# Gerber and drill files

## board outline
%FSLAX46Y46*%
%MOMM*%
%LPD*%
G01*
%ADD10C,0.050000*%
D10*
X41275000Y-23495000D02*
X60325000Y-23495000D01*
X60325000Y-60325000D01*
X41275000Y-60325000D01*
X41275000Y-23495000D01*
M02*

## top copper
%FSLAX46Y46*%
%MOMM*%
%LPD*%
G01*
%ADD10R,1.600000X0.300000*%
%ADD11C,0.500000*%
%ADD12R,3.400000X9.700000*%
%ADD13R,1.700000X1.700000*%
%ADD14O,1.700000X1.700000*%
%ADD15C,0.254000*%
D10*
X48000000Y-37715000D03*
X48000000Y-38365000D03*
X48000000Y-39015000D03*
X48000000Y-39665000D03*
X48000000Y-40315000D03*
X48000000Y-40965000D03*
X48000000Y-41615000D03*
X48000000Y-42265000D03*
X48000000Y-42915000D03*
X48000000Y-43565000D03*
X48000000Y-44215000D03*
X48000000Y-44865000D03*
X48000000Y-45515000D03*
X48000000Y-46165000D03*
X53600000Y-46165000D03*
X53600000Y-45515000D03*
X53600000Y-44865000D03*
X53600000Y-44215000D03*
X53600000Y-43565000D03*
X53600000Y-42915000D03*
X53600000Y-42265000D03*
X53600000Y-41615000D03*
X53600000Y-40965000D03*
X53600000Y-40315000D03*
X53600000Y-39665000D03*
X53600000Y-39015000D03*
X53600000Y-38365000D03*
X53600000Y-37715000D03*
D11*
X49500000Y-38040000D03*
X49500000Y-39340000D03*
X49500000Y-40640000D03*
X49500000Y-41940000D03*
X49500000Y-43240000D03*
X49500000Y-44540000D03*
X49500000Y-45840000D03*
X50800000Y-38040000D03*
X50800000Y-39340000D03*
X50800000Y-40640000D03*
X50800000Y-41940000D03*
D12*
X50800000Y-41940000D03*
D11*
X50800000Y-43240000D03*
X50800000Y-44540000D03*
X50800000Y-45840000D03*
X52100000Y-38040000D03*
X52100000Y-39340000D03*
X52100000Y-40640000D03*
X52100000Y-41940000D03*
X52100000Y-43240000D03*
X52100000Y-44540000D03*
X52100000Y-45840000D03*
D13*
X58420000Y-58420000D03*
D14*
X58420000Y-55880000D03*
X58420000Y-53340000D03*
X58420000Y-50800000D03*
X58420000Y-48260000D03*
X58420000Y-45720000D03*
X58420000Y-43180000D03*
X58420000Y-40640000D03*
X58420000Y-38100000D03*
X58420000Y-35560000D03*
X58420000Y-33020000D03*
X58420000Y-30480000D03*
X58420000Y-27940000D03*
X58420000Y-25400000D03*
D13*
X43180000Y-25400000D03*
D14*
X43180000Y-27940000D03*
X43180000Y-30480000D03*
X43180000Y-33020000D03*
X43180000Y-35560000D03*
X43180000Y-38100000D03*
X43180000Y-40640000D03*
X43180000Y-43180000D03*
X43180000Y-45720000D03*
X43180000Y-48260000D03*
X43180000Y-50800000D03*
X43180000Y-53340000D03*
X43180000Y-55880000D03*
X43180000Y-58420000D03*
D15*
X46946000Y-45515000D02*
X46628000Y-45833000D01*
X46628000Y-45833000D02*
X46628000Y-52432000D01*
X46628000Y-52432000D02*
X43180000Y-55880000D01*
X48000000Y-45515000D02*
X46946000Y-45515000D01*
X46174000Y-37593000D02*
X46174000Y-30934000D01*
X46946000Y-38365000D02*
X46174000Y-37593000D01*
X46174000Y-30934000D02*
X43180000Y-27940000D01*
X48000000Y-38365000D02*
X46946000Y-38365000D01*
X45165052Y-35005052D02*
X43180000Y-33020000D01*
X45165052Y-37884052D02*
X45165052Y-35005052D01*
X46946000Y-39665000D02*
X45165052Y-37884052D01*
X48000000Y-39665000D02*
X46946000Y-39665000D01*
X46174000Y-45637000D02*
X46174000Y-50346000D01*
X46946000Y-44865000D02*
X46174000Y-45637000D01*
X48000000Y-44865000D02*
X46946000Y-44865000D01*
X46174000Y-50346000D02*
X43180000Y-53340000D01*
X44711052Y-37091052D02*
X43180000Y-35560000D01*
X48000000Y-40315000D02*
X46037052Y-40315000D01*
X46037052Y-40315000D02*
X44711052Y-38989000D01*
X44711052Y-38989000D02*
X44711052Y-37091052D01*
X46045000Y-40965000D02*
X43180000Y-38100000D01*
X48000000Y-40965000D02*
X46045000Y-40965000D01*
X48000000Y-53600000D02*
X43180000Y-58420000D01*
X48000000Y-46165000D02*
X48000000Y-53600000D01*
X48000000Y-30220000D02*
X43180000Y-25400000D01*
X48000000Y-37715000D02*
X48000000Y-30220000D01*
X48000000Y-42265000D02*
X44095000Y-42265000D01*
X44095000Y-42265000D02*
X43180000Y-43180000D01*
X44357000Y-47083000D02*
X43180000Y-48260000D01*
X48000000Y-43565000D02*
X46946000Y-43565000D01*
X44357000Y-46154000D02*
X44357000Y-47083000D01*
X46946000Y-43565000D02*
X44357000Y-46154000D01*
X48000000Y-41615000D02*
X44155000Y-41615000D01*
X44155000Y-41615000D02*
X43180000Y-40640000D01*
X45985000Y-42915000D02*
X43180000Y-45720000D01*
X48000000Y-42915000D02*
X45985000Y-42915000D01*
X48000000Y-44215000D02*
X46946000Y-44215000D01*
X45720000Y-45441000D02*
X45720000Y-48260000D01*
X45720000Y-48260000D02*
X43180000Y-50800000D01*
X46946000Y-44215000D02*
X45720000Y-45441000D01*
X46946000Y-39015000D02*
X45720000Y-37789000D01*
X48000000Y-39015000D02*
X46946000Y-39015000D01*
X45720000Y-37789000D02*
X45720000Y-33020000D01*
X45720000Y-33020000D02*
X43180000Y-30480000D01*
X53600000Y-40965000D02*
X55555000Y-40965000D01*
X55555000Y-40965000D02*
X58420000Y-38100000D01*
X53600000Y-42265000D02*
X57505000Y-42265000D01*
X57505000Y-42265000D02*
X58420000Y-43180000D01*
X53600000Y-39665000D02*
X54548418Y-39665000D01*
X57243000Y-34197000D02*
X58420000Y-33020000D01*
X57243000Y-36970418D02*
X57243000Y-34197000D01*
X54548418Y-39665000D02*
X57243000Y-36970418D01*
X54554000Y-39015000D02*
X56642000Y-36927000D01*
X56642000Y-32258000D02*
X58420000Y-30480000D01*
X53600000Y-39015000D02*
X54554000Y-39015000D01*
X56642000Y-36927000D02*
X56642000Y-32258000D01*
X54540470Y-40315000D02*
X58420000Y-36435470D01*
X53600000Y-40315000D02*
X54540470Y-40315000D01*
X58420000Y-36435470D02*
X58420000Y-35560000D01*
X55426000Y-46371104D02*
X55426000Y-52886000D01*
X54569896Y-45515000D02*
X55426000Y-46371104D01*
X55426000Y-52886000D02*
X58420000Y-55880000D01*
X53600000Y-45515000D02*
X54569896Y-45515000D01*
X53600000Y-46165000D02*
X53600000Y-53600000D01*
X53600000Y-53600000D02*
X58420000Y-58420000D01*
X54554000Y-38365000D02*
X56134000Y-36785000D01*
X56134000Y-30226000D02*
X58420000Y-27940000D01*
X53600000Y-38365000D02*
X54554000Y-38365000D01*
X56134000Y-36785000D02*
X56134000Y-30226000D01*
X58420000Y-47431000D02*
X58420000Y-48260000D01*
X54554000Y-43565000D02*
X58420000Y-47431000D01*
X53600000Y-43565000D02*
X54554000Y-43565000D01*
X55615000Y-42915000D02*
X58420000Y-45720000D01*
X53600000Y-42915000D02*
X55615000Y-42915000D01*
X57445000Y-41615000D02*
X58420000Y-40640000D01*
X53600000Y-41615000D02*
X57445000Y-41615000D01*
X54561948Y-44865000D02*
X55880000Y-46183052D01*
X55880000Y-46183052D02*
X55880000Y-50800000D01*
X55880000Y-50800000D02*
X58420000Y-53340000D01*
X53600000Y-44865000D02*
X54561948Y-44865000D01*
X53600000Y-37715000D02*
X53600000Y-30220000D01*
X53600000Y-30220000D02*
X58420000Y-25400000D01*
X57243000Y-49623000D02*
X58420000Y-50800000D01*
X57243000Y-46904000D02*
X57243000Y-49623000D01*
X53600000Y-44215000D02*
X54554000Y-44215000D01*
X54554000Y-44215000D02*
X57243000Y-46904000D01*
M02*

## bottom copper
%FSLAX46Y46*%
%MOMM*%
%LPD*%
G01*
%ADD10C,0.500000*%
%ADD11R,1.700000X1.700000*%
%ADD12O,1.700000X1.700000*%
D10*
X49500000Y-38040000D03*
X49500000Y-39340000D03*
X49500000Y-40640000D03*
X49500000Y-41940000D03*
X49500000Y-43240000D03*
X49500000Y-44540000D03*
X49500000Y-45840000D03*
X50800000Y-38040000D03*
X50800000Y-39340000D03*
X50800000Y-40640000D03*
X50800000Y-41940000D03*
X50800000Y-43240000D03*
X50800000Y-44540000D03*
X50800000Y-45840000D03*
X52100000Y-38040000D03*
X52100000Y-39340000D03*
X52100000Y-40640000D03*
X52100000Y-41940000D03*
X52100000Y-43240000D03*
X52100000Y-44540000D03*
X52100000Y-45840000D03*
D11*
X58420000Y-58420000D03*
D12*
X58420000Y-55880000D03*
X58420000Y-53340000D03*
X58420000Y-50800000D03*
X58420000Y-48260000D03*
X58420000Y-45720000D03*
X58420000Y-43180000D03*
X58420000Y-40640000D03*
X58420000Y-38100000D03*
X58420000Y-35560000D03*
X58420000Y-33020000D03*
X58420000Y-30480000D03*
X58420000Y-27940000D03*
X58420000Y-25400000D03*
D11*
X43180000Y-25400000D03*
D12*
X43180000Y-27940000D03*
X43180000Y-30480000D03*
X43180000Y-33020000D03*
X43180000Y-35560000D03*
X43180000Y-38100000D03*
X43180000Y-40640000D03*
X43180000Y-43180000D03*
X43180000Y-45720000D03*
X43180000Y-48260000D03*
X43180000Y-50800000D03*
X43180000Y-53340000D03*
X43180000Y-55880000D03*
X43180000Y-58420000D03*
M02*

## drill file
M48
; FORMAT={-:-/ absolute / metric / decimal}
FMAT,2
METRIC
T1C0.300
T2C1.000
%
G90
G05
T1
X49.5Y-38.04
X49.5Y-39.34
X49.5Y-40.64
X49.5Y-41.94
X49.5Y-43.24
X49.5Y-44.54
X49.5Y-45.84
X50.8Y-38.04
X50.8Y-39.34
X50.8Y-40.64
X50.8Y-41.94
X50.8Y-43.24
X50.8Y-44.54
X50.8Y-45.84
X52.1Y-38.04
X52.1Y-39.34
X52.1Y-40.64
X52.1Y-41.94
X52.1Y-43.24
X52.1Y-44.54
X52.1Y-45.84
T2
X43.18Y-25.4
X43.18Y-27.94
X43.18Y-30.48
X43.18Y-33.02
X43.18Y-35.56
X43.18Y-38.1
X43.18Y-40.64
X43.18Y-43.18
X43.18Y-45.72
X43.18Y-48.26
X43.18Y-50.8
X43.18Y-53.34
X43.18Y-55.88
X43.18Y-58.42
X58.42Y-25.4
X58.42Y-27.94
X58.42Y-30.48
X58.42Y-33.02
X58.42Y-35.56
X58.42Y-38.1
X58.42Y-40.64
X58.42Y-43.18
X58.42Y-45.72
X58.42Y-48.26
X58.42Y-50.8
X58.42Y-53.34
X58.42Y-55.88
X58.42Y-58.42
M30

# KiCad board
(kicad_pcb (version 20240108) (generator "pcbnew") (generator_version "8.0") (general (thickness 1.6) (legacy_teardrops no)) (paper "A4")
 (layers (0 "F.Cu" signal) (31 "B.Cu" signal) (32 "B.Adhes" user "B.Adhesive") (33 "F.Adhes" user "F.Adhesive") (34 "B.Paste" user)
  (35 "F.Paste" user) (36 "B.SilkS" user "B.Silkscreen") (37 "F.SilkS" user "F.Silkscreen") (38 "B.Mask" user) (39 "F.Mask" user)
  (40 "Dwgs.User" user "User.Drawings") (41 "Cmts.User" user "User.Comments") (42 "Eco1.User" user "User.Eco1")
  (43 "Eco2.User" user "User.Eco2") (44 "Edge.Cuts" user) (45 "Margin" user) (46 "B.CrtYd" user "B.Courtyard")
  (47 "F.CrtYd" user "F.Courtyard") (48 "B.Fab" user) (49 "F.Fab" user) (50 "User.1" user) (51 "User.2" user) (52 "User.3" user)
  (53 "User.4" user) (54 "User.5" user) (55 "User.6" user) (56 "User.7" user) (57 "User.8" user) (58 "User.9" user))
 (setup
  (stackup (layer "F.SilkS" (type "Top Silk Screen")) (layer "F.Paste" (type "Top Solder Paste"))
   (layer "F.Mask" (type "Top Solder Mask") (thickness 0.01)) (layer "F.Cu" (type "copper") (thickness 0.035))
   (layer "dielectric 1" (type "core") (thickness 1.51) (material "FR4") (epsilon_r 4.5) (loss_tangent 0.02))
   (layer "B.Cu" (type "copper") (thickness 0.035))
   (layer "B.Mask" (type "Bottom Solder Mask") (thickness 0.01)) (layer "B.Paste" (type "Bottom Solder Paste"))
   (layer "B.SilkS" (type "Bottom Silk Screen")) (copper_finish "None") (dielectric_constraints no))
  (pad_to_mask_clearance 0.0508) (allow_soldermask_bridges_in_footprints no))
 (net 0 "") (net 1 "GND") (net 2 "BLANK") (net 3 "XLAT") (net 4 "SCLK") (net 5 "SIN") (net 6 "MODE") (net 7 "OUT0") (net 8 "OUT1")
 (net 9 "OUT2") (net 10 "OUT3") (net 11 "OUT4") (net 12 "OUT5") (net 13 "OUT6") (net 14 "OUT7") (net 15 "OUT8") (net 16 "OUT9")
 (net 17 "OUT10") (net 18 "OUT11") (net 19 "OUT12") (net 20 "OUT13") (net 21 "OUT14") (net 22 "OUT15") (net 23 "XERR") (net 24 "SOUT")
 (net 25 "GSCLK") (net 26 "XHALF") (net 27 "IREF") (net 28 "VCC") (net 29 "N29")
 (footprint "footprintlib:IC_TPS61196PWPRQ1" (layer "F.Cu") (at 50.8 41.94)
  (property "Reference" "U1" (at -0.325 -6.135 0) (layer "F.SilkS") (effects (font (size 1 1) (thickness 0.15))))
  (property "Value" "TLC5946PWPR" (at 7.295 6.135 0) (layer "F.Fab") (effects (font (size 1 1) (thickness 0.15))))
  (pad "1" smd rect (at -2.8 -4.225) (size 1.6 0.3) (layers "F.Cu") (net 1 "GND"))
  (pad "2" smd rect (at -2.8 -3.575) (size 1.6 0.3) (layers "F.Cu") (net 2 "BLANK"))
  (pad "3" smd rect (at -2.8 -2.925) (size 1.6 0.3) (layers "F.Cu") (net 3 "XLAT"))
  (pad "4" smd rect (at -2.8 -2.275) (size 1.6 0.3) (layers "F.Cu") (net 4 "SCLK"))
  (pad "5" smd rect (at -2.8 -1.625) (size 1.6 0.3) (layers "F.Cu") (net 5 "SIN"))
  (pad "6" smd rect (at -2.8 -0.975) (size 1.6 0.3) (layers "F.Cu") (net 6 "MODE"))
  (pad "7" smd rect (at -2.8 -0.325) (size 1.6 0.3) (layers "F.Cu") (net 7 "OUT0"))
  (pad "8" smd rect (at -2.8 0.325) (size 1.6 0.3) (layers "F.Cu") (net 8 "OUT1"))
  (pad "9" smd rect (at -2.8 0.975) (size 1.6 0.3) (layers "F.Cu") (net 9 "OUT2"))
  (pad "10" smd rect (at -2.8 1.625) (size 1.6 0.3) (layers "F.Cu") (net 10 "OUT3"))
  (pad "11" smd rect (at -2.8 2.275) (size 1.6 0.3) (layers "F.Cu") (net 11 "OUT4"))
  (pad "12" smd rect (at -2.8 2.925) (size 1.6 0.3) (layers "F.Cu") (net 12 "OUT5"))
  (pad "13" smd rect (at -2.8 3.575) (size 1.6 0.3) (layers "F.Cu") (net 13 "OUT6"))
  (pad "14" smd rect (at -2.8 4.225) (size 1.6 0.3) (layers "F.Cu") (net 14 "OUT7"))
  (pad "15" smd rect (at 2.8 4.225) (size 1.6 0.3) (layers "F.Cu") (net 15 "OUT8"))
  (pad "16" smd rect (at 2.8 3.575) (size 1.6 0.3) (layers "F.Cu") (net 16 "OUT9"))
  (pad "17" smd rect (at 2.8 2.925) (size 1.6 0.3) (layers "F.Cu") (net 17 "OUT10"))
  (pad "18" smd rect (at 2.8 2.275) (size 1.6 0.3) (layers "F.Cu") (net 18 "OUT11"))
  (pad "19" smd rect (at 2.8 1.625) (size 1.6 0.3) (layers "F.Cu") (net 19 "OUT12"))
  (pad "20" smd rect (at 2.8 0.975) (size 1.6 0.3) (layers "F.Cu") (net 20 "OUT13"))
  (pad "21" smd rect (at 2.8 0.325) (size 1.6 0.3) (layers "F.Cu") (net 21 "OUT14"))
  (pad "22" smd rect (at 2.8 -0.325) (size 1.6 0.3) (layers "F.Cu") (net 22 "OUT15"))
  (pad "23" smd rect (at 2.8 -0.975) (size 1.6 0.3) (layers "F.Cu") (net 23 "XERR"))
  (pad "24" smd rect (at 2.8 -1.625) (size 1.6 0.3) (layers "F.Cu") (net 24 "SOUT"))
  (pad "25" smd rect (at 2.8 -2.275) (size 1.6 0.3) (layers "F.Cu") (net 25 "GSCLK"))
  (pad "26" smd rect (at 2.8 -2.925) (size 1.6 0.3) (layers "F.Cu") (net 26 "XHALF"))
  (pad "27" smd rect (at 2.8 -3.575) (size 1.6 0.3) (layers "F.Cu") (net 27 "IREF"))
  (pad "28" smd rect (at 2.8 -4.225) (size 1.6 0.3) (layers "F.Cu") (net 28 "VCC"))
  (pad "29" thru_hole circle (at -1.3 -3.9) (size 0.5 0.5) (drill 0.3) (layers "*.Cu") (remove_unused_layers no) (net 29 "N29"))
  (pad "29" thru_hole circle (at -1.3 -2.6) (size 0.5 0.5) (drill 0.3) (layers "*.Cu") (remove_unused_layers no) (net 29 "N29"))
  (pad "29" thru_hole circle (at -1.3 -1.3) (size 0.5 0.5) (drill 0.3) (layers "*.Cu") (remove_unused_layers no) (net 29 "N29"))
  (pad "29" thru_hole circle (at -1.3 0) (size 0.5 0.5) (drill 0.3) (layers "*.Cu") (remove_unused_layers no) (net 29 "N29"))
  (pad "29" thru_hole circle (at -1.3 1.3) (size 0.5 0.5) (drill 0.3) (layers "*.Cu") (remove_unused_layers no) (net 29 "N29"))
  (pad "29" thru_hole circle (at -1.3 2.6) (size 0.5 0.5) (drill 0.3) (layers "*.Cu") (remove_unused_layers no) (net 29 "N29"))
  (pad "29" thru_hole circle (at -1.3 3.9) (size 0.5 0.5) (drill 0.3) (layers "*.Cu") (remove_unused_layers no) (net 29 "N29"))
  (pad "29" thru_hole circle (at 0 -3.9) (size 0.5 0.5) (drill 0.3) (layers "*.Cu") (remove_unused_layers no) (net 29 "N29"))
  (pad "29" thru_hole circle (at 0 -2.6) (size 0.5 0.5) (drill 0.3) (layers "*.Cu") (remove_unused_layers no) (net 29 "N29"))
  (pad "29" thru_hole circle (at 0 -1.3) (size 0.5 0.5) (drill 0.3) (layers "*.Cu") (remove_unused_layers no) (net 29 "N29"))
  (pad "29" thru_hole circle (at 0 0) (size 0.5 0.5) (drill 0.3) (layers "*.Cu") (remove_unused_layers no) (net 29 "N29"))
  (pad "29" smd rect (at 0 0) (size 3.4 9.7) (layers "F.Cu") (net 29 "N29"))
  (pad "29" thru_hole circle (at 0 1.3) (size 0.5 0.5) (drill 0.3) (layers "*.Cu") (remove_unused_layers no) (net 29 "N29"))
  (pad "29" thru_hole circle (at 0 2.6) (size 0.5 0.5) (drill 0.3) (layers "*.Cu") (remove_unused_layers no) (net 29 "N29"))
  (pad "29" thru_hole circle (at 0 3.9) (size 0.5 0.5) (drill 0.3) (layers "*.Cu") (remove_unused_layers no) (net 29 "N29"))
  (pad "29" thru_hole circle (at 1.3 -3.9) (size 0.5 0.5) (drill 0.3) (layers "*.Cu") (remove_unused_layers no) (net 29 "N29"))
  (pad "29" thru_hole circle (at 1.3 -2.6) (size 0.5 0.5) (drill 0.3) (layers "*.Cu") (remove_unused_layers no) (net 29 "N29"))
  (pad "29" thru_hole circle (at 1.3 -1.3) (size 0.5 0.5) (drill 0.3) (layers "*.Cu") (remove_unused_layers no) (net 29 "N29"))
  (pad "29" thru_hole circle (at 1.3 0) (size 0.5 0.5) (drill 0.3) (layers "*.Cu") (remove_unused_layers no) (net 29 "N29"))
  (pad "29" thru_hole circle (at 1.3 1.3) (size 0.5 0.5) (drill 0.3) (layers "*.Cu") (remove_unused_layers no) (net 29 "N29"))
  (pad "29" thru_hole circle (at 1.3 2.6) (size 0.5 0.5) (drill 0.3) (layers "*.Cu") (remove_unused_layers no) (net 29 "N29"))
  (pad "29" thru_hole circle (at 1.3 3.9) (size 0.5 0.5) (drill 0.3) (layers "*.Cu") (remove_unused_layers no) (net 29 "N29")))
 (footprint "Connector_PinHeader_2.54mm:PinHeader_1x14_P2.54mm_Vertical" (layer "F.Cu") (at 58.42 58.42 180)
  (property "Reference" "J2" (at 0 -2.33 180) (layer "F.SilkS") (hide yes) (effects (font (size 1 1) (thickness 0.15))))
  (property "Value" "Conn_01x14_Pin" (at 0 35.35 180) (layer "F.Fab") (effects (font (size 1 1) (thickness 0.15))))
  (pad "1" thru_hole rect (at 0 0 180) (size 1.7 1.7) (drill 1) (layers "*.Cu" "*.Mask") (remove_unused_layers no) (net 15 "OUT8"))
  (pad "2" thru_hole oval (at 0 2.54 180) (size 1.7 1.7) (drill 1) (layers "*.Cu" "*.Mask") (remove_unused_layers no) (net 16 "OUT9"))
  (pad "3" thru_hole oval (at 0 5.08 180) (size 1.7 1.7) (drill 1) (layers "*.Cu" "*.Mask") (remove_unused_layers no) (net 17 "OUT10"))
  (pad "4" thru_hole oval (at 0 7.62 180) (size 1.7 1.7) (drill 1) (layers "*.Cu" "*.Mask") (remove_unused_layers no) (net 18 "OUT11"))
  (pad "5" thru_hole oval (at 0 10.16 180) (size 1.7 1.7) (drill 1) (layers "*.Cu" "*.Mask") (remove_unused_layers no) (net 19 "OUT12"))
  (pad "6" thru_hole oval (at 0 12.7 180) (size 1.7 1.7) (drill 1) (layers "*.Cu" "*.Mask") (remove_unused_layers no) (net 20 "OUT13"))
  (pad "7" thru_hole oval (at 0 15.24 180) (size 1.7 1.7) (drill 1) (layers "*.Cu" "*.Mask") (remove_unused_layers no) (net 21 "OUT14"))
  (pad "8" thru_hole oval (at 0 17.78 180) (size 1.7 1.7) (drill 1) (layers "*.Cu" "*.Mask") (remove_unused_layers no) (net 22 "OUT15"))
  (pad "9" thru_hole oval (at 0 20.32 180) (size 1.7 1.7) (drill 1) (layers "*.Cu" "*.Mask") (remove_unused_layers no) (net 23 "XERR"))
  (pad "10" thru_hole oval (at 0 22.86 180) (size 1.7 1.7) (drill 1) (layers "*.Cu" "*.Mask") (remove_unused_layers no) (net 24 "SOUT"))
  (pad "11" thru_hole oval (at 0 25.4 180) (size 1.7 1.7) (drill 1) (layers "*.Cu" "*.Mask") (remove_unused_layers no) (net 25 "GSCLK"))
  (pad "12" thru_hole oval (at 0 27.94 180) (size 1.7 1.7) (drill 1) (layers "*.Cu" "*.Mask") (remove_unused_layers no) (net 26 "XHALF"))
  (pad "13" thru_hole oval (at 0 30.48 180) (size 1.7 1.7) (drill 1) (layers "*.Cu" "*.Mask") (remove_unused_layers no) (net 27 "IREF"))
  (pad "14" thru_hole oval (at 0 33.02 180) (size 1.7 1.7) (drill 1) (layers "*.Cu" "*.Mask") (remove_unused_layers no) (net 28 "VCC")))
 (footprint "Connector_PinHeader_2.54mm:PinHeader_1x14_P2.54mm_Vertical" (layer "F.Cu") (at 43.18 25.4)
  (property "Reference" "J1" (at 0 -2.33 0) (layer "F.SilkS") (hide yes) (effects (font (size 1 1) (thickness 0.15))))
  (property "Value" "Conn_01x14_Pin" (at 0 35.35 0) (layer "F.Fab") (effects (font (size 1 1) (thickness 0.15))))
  (pad "1" thru_hole rect (at 0 0) (size 1.7 1.7) (drill 1) (layers "*.Cu" "*.Mask") (remove_unused_layers no) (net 1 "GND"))
  (pad "2" thru_hole oval (at 0 2.54) (size 1.7 1.7) (drill 1) (layers "*.Cu" "*.Mask") (remove_unused_layers no) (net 2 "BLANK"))
  (pad "3" thru_hole oval (at 0 5.08) (size 1.7 1.7) (drill 1) (layers "*.Cu" "*.Mask") (remove_unused_layers no) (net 3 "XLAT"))
  (pad "4" thru_hole oval (at 0 7.62) (size 1.7 1.7) (drill 1) (layers "*.Cu" "*.Mask") (remove_unused_layers no) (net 4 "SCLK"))
  (pad "5" thru_hole oval (at 0 10.16) (size 1.7 1.7) (drill 1) (layers "*.Cu" "*.Mask") (remove_unused_layers no) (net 5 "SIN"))
  (pad "6" thru_hole oval (at 0 12.7) (size 1.7 1.7) (drill 1) (layers "*.Cu" "*.Mask") (remove_unused_layers no) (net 6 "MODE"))
  (pad "7" thru_hole oval (at 0 15.24) (size 1.7 1.7) (drill 1) (layers "*.Cu" "*.Mask") (remove_unused_layers no) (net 7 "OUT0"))
  (pad "8" thru_hole oval (at 0 17.78) (size 1.7 1.7) (drill 1) (layers "*.Cu" "*.Mask") (remove_unused_layers no) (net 8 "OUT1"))
  (pad "9" thru_hole oval (at 0 20.32) (size 1.7 1.7) (drill 1) (layers "*.Cu" "*.Mask") (remove_unused_layers no) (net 9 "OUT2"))
  (pad "10" thru_hole oval (at 0 22.86) (size 1.7 1.7) (drill 1) (layers "*.Cu" "*.Mask") (remove_unused_layers no) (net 10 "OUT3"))
  (pad "11" thru_hole oval (at 0 25.4) (size 1.7 1.7) (drill 1) (layers "*.Cu" "*.Mask") (remove_unused_layers no) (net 11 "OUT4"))
  (pad "12" thru_hole oval (at 0 27.94) (size 1.7 1.7) (drill 1) (layers "*.Cu" "*.Mask") (remove_unused_layers no) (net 12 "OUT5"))
  (pad "13" thru_hole oval (at 0 30.48) (size 1.7 1.7) (drill 1) (layers "*.Cu" "*.Mask") (remove_unused_layers no) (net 13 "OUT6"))
  (pad "14" thru_hole oval (at 0 33.02) (size 1.7 1.7) (drill 1) (layers "*.Cu" "*.Mask") (remove_unused_layers no) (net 14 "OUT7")))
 (gr_rect (start 41.275 23.495) (end 60.325 60.325) (stroke (width 0.05) (type default)) (fill none) (layer "Edge.Cuts"))
 (segment (start 46.946 45.515) (end 46.628 45.833) (width 0.254) (layer "F.Cu") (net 13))
 (segment (start 46.628 45.833) (end 46.628 52.432) (width 0.254) (layer "F.Cu") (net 13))
 (segment (start 46.628 52.432) (end 43.18 55.88) (width 0.254) (layer "F.Cu") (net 13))
 (segment (start 48 45.515) (end 46.946 45.515) (width 0.254) (layer "F.Cu") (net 13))
 (segment (start 46.174 37.593) (end 46.174 30.934) (width 0.254) (layer "F.Cu") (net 2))
 (segment (start 46.946 38.365) (end 46.174 37.593) (width 0.254) (layer "F.Cu") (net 2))
 (segment (start 46.174 30.934) (end 43.18 27.94) (width 0.254) (layer "F.Cu") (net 2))
 (segment (start 48 38.365) (end 46.946 38.365) (width 0.254) (layer "F.Cu") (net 2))
 (segment (start 45.165052 35.005052) (end 43.18 33.02) (width 0.254) (layer "F.Cu") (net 4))
 (segment (start 45.165052 37.884052) (end 45.165052 35.005052) (width 0.254) (layer "F.Cu") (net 4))
 (segment (start 46.946 39.665) (end 45.165052 37.884052) (width 0.254) (layer "F.Cu") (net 4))
 (segment (start 48 39.665) (end 46.946 39.665) (width 0.254) (layer "F.Cu") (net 4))
 (segment (start 46.174 45.637) (end 46.174 50.346) (width 0.254) (layer "F.Cu") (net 12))
 (segment (start 46.946 44.865) (end 46.174 45.637) (width 0.254) (layer "F.Cu") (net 12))
 (segment (start 48 44.865) (end 46.946 44.865) (width 0.254) (layer "F.Cu") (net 12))
 (segment (start 46.174 50.346) (end 43.18 53.34) (width 0.254) (layer "F.Cu") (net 12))
 (segment (start 44.711052 37.091052) (end 43.18 35.56) (width 0.254) (layer "F.Cu") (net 5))
 (segment (start 48 40.315) (end 46.037052 40.315) (width 0.254) (layer "F.Cu") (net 5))
 (segment (start 46.037052 40.315) (end 44.711052 38.989) (width 0.254) (layer "F.Cu") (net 5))
 (segment (start 44.711052 38.989) (end 44.711052 37.091052) (width 0.254) (layer "F.Cu") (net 5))
 (segment (start 46.045 40.965) (end 43.18 38.1) (width 0.254) (layer "F.Cu") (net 6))
 (segment (start 48 40.965) (end 46.045 40.965) (width 0.254) (layer "F.Cu") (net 6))
 (segment (start 48 53.6) (end 43.18 58.42) (width 0.254) (layer "F.Cu") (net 14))
 (segment (start 48 46.165) (end 48 53.6) (width 0.254) (layer "F.Cu") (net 14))
 (segment (start 48 30.22) (end 43.18 25.4) (width 0.254) (layer "F.Cu") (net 1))
 (segment (start 48 37.715) (end 48 30.22) (width 0.254) (layer "F.Cu") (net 1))
 (segment (start 48 42.265) (end 44.095 42.265) (width 0.254) (layer "F.Cu") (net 8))
 (segment (start 44.095 42.265) (end 43.18 43.18) (width 0.254) (layer "F.Cu") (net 8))
 (segment (start 44.357 47.083) (end 43.18 48.26) (width 0.254) (layer "F.Cu") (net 10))
 (segment (start 48 43.565) (end 46.946 43.565) (width 0.254) (layer "F.Cu") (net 10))
 (segment (start 44.357 46.154) (end 44.357 47.083) (width 0.254) (layer "F.Cu") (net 10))
 (segment (start 46.946 43.565) (end 44.357 46.154) (width 0.254) (layer "F.Cu") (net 10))
 (segment (start 48 41.615) (end 44.155 41.615) (width 0.254) (layer "F.Cu") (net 7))
 (segment (start 44.155 41.615) (end 43.18 40.64) (width 0.254) (layer "F.Cu") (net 7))
 (segment (start 45.985 42.915) (end 43.18 45.72) (width 0.254) (layer "F.Cu") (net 9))
 (segment (start 48 42.915) (end 45.985 42.915) (width 0.254) (layer "F.Cu") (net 9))
 (segment (start 48 44.215) (end 46.946 44.215) (width 0.254) (layer "F.Cu") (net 11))
 (segment (start 45.72 45.441) (end 45.72 48.26) (width 0.254) (layer "F.Cu") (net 11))
 (segment (start 45.72 48.26) (end 43.18 50.8) (width 0.254) (layer "F.Cu") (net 11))
 (segment (start 46.946 44.215) (end 45.72 45.441) (width 0.254) (layer "F.Cu") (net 11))
 (segment (start 46.946 39.015) (end 45.72 37.789) (width 0.254) (layer "F.Cu") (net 3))
 (segment (start 48 39.015) (end 46.946 39.015) (width 0.254) (layer "F.Cu") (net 3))
 (segment (start 45.72 37.789) (end 45.72 33.02) (width 0.254) (layer "F.Cu") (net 3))
 (segment (start 45.72 33.02) (end 43.18 30.48) (width 0.254) (layer "F.Cu") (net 3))
 (segment (start 53.6 40.965) (end 55.555 40.965) (width 0.254) (layer "F.Cu") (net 23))
 (segment (start 55.555 40.965) (end 58.42 38.1) (width 0.254) (layer "F.Cu") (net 23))
 (segment (start 53.6 42.265) (end 57.505 42.265) (width 0.254) (layer "F.Cu") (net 21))
 (segment (start 57.505 42.265) (end 58.42 43.18) (width 0.254) (layer "F.Cu") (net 21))
 (segment (start 53.6 39.665) (end 54.548418 39.665) (width 0.254) (layer "F.Cu") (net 25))
 (segment (start 57.243 34.197) (end 58.42 33.02) (width 0.254) (layer "F.Cu") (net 25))
 (segment (start 57.243 36.970418) (end 57.243 34.197) (width 0.254) (layer "F.Cu") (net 25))
 (segment (start 54.548418 39.665) (end 57.243 36.970418) (width 0.254) (layer "F.Cu") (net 25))
 (segment (start 54.554 39.015) (end 56.642 36.927) (width 0.254) (layer "F.Cu") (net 26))
 (segment (start 56.642 32.258) (end 58.42 30.48) (width 0.254) (layer "F.Cu") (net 26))
 (segment (start 53.6 39.015) (end 54.554 39.015) (width 0.254) (layer "F.Cu") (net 26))
 (segment (start 56.642 36.927) (end 56.642 32.258) (width 0.254) (layer "F.Cu") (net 26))
 (segment (start 54.54047 40.315) (end 58.42 36.43547) (width 0.254) (layer "F.Cu") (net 24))
 (segment (start 53.6 40.315) (end 54.54047 40.315) (width 0.254) (layer "F.Cu") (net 24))
 (segment (start 58.42 36.43547) (end 58.42 35.56) (width 0.254) (layer "F.Cu") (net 24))
 (segment (start 55.426 46.371104) (end 55.426 52.886) (width 0.254) (layer "F.Cu") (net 16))
 (segment (start 54.569896 45.515) (end 55.426 46.371104) (width 0.254) (layer "F.Cu") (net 16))
 (segment (start 55.426 52.886) (end 58.42 55.88) (width 0.254) (layer "F.Cu") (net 16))
 (segment (start 53.6 45.515) (end 54.569896 45.515) (width 0.254) (layer "F.Cu") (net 16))
 (segment (start 53.6 46.165) (end 53.6 53.6) (width 0.254) (layer "F.Cu") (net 15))
 (segment (start 53.6 53.6) (end 58.42 58.42) (width 0.254) (layer "F.Cu") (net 15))
 (segment (start 54.554 38.365) (end 56.134 36.785) (width 0.254) (layer "F.Cu") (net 27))
 (segment (start 56.134 30.226) (end 58.42 27.94) (width 0.254) (layer "F.Cu") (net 27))
 (segment (start 53.6 38.365) (end 54.554 38.365) (width 0.254) (layer "F.Cu") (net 27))
 (segment (start 56.134 36.785) (end 56.134 30.226) (width 0.254) (layer "F.Cu") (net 27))
 (segment (start 58.42 47.431) (end 58.42 48.26) (width 0.254) (layer "F.Cu") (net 19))
 (segment (start 54.554 43.565) (end 58.42 47.431) (width 0.254) (layer "F.Cu") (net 19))
 (segment (start 53.6 43.565) (end 54.554 43.565) (width 0.254) (layer "F.Cu") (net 19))
 (segment (start 55.615 42.915) (end 58.42 45.72) (width 0.254) (layer "F.Cu") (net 20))
 (segment (start 53.6 42.915) (end 55.615 42.915) (width 0.254) (layer "F.Cu") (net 20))
 (segment (start 57.445 41.615) (end 58.42 40.64) (width 0.254) (layer "F.Cu") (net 22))
 (segment (start 53.6 41.615) (end 57.445 41.615) (width 0.254) (layer "F.Cu") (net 22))
 (segment (start 54.561948 44.865) (end 55.88 46.183052) (width 0.254) (layer "F.Cu") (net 17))
 (segment (start 55.88 46.183052) (end 55.88 50.8) (width 0.254) (layer "F.Cu") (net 17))
 (segment (start 55.88 50.8) (end 58.42 53.34) (width 0.254) (layer "F.Cu") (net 17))
 (segment (start 53.6 44.865) (end 54.561948 44.865) (width 0.254) (layer "F.Cu") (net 17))
 (segment (start 53.6 37.715) (end 53.6 30.22) (width 0.254) (layer "F.Cu") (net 28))
 (segment (start 53.6 30.22) (end 58.42 25.4) (width 0.254) (layer "F.Cu") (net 28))
 (segment (start 57.243 49.623) (end 58.42 50.8) (width 0.254) (layer "F.Cu") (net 18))
 (segment (start 57.243 46.904) (end 57.243 49.623) (width 0.254) (layer "F.Cu") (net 18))
 (segment (start 53.6 44.215) (end 54.554 44.215) (width 0.254) (layer "F.Cu") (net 18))
 (segment (start 54.554 44.215) (end 57.243 46.904) (width 0.254) (layer "F.Cu") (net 18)))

